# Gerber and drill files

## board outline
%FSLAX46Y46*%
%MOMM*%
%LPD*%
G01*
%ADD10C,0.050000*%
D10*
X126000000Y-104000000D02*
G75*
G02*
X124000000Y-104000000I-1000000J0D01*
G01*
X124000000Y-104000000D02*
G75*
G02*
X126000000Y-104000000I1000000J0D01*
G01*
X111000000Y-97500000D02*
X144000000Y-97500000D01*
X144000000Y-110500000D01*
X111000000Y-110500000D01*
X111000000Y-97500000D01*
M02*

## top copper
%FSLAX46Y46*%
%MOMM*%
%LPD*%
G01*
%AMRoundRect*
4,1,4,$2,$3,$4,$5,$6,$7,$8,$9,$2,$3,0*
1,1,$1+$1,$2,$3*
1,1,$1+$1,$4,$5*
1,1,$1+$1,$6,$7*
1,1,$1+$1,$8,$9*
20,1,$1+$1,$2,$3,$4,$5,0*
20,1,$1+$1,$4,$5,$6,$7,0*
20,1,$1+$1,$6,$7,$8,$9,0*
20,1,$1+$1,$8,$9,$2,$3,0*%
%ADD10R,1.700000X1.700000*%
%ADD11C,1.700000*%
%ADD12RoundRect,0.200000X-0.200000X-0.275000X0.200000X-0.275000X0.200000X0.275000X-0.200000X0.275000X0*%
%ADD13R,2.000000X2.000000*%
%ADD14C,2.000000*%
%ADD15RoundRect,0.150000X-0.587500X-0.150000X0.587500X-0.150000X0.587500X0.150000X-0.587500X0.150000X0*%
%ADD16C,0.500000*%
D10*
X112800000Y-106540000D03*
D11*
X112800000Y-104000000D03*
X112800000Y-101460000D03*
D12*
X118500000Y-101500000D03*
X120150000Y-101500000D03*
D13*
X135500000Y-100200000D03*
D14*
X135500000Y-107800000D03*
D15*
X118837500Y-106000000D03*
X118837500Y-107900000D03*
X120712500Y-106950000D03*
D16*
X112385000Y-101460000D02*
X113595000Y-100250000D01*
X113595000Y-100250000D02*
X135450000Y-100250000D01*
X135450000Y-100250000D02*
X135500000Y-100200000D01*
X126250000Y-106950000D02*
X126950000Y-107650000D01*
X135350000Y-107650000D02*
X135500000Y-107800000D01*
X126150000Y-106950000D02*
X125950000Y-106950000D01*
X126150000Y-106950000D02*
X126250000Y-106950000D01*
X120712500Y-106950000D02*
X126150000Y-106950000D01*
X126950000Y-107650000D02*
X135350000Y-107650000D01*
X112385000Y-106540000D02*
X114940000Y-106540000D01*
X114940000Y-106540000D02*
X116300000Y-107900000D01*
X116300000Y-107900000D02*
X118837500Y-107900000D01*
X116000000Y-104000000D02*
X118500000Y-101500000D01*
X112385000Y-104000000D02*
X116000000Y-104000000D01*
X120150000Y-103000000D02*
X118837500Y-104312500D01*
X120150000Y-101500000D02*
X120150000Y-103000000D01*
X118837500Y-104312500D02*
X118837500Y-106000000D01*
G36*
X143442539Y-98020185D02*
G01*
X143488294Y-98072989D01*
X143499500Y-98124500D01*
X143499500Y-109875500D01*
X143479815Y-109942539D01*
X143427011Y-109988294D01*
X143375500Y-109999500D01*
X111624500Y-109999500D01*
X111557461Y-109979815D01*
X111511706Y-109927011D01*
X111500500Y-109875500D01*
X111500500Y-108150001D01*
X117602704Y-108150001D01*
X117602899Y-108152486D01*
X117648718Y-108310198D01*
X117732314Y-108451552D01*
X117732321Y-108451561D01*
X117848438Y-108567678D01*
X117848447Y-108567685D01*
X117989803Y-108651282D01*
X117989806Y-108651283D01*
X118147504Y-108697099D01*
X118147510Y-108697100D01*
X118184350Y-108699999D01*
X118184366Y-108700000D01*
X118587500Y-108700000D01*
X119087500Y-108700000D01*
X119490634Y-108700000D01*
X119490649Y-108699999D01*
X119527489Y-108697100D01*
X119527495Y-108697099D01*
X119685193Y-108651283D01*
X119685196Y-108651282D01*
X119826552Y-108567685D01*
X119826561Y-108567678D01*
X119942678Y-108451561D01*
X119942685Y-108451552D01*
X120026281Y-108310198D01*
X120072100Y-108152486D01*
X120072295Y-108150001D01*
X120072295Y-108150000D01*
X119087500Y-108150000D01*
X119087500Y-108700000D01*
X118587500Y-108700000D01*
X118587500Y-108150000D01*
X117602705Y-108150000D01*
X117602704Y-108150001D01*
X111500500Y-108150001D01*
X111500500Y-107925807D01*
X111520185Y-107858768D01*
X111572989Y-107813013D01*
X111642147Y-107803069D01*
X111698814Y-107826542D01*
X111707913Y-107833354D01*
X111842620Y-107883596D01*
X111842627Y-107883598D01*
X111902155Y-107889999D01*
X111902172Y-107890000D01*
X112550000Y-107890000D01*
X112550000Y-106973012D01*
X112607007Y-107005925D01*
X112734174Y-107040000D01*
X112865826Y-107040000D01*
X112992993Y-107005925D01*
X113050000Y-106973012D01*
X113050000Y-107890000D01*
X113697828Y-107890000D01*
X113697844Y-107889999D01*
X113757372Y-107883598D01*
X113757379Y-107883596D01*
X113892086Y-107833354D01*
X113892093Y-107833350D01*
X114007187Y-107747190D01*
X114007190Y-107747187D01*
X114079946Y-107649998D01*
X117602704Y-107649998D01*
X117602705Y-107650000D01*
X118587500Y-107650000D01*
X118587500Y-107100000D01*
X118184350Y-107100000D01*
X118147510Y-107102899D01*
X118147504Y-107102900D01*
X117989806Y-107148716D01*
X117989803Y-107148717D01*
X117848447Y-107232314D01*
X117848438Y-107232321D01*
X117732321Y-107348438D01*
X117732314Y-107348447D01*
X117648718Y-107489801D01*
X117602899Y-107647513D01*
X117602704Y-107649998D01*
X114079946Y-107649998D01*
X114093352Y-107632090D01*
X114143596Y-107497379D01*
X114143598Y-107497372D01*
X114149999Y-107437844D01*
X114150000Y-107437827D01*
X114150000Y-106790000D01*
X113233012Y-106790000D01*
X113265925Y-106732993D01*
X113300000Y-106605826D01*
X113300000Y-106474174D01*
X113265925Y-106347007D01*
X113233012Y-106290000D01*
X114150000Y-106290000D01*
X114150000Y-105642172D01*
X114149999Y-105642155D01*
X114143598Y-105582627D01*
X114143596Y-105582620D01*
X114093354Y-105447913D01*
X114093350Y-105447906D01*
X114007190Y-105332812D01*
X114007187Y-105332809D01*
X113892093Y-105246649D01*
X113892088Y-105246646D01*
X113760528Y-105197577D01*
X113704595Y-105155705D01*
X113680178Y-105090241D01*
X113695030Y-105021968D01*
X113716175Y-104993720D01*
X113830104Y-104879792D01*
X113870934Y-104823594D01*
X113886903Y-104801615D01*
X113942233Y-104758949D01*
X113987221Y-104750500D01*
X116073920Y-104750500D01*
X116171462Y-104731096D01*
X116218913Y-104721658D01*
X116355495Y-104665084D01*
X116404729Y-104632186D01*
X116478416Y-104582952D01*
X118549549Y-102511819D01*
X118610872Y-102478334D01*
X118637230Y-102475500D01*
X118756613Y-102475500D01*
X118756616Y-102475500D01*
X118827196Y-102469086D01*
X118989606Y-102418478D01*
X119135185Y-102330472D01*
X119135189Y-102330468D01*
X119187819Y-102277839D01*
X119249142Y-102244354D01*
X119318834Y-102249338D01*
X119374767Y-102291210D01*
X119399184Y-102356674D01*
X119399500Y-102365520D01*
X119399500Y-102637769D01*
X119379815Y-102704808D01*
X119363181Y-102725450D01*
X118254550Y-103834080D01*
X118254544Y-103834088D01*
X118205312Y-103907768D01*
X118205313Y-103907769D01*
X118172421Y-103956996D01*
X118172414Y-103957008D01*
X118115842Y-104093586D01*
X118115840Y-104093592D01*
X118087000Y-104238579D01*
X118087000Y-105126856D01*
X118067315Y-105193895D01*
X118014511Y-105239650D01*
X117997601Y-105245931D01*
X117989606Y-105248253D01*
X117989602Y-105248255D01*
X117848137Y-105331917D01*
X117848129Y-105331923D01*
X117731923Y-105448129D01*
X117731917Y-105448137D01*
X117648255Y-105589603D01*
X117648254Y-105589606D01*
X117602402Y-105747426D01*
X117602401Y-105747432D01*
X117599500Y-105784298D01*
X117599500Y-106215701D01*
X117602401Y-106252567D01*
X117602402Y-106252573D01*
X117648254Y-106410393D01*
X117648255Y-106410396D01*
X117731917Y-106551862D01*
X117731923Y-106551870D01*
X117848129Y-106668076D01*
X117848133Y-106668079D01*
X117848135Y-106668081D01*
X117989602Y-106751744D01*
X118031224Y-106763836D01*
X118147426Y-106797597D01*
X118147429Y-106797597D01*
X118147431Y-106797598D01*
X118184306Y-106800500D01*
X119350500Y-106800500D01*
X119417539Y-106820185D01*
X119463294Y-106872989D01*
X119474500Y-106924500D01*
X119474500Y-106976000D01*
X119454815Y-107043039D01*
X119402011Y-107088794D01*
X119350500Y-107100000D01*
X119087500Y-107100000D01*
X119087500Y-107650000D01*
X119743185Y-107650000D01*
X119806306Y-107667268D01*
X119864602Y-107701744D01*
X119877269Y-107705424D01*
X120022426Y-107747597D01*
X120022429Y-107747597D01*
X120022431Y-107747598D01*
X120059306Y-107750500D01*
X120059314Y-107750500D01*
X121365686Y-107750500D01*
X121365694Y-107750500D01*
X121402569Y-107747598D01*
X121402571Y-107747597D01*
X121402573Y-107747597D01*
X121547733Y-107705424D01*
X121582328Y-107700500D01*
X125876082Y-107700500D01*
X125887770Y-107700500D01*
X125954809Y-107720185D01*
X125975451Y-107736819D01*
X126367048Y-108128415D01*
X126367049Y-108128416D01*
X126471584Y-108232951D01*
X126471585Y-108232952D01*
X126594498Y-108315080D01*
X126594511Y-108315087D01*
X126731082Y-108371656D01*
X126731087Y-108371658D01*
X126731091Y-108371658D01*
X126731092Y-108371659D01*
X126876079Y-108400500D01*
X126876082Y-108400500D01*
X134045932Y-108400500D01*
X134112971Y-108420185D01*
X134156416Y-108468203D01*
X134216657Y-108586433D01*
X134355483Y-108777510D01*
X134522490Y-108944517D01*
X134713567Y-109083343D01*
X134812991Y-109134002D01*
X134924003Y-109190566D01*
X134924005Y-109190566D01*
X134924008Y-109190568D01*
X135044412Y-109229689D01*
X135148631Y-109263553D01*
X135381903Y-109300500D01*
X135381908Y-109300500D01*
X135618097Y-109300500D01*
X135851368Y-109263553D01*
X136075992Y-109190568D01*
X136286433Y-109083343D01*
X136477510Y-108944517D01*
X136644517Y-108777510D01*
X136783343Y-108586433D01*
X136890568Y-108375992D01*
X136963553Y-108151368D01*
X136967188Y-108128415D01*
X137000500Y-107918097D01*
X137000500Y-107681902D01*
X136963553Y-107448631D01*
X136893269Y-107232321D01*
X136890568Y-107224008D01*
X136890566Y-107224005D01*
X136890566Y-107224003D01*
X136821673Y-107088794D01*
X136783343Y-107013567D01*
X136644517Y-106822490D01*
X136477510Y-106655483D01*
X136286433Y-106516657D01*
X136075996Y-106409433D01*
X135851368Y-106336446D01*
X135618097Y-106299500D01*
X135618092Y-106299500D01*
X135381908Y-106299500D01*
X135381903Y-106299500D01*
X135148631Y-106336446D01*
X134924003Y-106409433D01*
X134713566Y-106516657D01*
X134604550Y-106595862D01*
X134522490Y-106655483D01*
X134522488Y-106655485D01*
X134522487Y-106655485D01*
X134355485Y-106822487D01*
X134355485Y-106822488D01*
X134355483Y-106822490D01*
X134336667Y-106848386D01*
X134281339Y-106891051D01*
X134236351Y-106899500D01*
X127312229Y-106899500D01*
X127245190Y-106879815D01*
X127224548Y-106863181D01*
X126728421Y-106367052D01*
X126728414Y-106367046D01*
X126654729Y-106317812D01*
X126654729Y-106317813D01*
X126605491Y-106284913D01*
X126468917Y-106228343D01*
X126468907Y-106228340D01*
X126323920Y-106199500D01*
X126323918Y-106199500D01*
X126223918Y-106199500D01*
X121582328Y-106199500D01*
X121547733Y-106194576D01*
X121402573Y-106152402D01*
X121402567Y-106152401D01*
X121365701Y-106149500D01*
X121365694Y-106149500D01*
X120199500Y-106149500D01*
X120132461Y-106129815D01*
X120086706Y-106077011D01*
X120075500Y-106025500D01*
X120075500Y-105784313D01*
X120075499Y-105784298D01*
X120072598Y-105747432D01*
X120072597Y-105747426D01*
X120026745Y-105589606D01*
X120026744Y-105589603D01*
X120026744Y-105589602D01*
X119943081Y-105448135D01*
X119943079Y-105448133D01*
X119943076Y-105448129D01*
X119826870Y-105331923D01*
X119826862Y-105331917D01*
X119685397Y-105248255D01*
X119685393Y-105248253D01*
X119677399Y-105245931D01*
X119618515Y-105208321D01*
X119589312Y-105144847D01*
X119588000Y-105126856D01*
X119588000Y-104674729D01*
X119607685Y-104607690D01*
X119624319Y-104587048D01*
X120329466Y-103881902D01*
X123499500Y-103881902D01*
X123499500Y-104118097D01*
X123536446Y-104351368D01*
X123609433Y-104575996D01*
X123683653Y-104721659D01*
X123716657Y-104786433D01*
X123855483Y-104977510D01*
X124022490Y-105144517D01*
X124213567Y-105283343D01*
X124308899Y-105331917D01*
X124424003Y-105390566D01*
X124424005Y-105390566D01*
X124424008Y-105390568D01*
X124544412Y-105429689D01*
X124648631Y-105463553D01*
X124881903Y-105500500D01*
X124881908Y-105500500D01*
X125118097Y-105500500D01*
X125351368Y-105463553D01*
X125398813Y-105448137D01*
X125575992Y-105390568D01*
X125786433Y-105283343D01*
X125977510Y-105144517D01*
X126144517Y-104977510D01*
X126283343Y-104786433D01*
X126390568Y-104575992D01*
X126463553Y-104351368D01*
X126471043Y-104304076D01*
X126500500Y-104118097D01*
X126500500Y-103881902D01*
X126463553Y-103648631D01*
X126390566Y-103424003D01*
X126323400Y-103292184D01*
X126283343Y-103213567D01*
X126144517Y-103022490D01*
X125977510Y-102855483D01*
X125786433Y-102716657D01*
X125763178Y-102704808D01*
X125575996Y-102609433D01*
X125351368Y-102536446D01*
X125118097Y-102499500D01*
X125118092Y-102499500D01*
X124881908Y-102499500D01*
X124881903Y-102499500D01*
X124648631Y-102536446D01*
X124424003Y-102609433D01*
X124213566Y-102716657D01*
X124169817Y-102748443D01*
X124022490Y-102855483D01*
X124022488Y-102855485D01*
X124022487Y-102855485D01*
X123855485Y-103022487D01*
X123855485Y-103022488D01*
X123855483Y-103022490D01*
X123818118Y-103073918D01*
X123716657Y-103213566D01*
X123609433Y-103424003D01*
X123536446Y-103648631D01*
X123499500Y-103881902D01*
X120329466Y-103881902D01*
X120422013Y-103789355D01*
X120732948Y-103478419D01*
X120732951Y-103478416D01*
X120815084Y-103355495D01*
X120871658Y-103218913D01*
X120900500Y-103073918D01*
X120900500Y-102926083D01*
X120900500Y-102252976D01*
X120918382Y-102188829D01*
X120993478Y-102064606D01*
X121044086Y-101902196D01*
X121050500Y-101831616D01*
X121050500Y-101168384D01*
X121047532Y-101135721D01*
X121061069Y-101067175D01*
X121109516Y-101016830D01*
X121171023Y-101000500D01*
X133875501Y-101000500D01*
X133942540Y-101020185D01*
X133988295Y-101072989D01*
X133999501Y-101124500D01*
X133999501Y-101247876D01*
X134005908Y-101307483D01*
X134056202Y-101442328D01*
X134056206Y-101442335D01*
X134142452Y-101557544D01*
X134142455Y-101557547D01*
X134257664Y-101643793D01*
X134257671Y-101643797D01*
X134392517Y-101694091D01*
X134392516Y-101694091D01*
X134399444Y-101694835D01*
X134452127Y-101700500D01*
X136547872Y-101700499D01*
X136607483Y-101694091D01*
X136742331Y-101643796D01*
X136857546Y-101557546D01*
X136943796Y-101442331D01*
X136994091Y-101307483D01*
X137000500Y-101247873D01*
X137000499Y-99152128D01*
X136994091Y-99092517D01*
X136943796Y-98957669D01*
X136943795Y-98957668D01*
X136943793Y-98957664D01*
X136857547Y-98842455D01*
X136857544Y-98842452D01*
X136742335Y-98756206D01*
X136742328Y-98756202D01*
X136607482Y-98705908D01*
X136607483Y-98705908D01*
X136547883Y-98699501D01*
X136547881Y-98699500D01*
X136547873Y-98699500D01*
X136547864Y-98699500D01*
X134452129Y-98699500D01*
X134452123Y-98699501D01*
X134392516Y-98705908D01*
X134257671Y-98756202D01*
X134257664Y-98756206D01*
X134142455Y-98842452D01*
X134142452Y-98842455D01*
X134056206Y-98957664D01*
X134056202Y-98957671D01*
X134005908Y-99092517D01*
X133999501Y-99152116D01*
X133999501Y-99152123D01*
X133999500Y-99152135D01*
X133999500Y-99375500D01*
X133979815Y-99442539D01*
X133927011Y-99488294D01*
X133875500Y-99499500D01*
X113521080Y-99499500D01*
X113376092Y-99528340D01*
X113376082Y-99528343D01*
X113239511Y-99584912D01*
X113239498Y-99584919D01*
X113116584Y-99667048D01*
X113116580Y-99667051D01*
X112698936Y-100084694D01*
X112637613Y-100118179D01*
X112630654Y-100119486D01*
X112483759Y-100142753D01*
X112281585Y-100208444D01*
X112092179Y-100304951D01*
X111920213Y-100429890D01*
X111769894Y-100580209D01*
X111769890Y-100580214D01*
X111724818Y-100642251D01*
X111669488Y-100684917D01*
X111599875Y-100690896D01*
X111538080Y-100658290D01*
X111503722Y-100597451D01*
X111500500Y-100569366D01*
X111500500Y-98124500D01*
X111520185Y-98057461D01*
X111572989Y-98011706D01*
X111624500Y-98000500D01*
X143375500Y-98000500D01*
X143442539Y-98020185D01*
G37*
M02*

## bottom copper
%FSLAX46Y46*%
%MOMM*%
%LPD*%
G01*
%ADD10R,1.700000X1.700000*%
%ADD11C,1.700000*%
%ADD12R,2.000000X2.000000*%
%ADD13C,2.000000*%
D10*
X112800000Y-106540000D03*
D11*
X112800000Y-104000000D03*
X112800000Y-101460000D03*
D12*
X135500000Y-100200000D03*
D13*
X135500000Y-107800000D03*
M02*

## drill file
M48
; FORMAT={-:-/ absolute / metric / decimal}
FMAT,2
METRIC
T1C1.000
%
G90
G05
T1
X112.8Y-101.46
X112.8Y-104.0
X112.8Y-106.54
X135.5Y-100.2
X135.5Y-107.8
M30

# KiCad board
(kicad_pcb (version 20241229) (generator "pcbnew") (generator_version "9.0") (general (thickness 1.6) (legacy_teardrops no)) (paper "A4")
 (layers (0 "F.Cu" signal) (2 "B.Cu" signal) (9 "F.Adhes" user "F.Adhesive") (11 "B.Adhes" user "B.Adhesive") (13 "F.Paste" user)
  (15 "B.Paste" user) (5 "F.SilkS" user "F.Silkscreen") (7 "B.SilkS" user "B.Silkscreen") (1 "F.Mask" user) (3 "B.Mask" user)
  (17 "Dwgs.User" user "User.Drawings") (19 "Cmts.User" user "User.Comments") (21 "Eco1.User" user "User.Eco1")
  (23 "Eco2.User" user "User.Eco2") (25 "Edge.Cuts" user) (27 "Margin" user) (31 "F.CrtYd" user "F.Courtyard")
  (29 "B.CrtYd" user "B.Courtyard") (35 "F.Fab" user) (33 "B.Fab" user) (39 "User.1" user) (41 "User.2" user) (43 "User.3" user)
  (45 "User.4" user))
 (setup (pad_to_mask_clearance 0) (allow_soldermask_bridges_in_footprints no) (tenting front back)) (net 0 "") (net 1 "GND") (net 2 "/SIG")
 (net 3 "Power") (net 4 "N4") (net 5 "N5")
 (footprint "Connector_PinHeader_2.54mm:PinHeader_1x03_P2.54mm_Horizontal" (layer "F.Cu") (at 112.8 106.54 180)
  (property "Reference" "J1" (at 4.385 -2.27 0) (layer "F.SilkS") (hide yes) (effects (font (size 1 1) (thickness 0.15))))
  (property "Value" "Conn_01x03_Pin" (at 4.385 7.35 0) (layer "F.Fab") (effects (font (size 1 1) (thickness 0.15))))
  (pad "1" thru_hole rect (at 0 0 180) (size 1.7 1.7) (drill 1) (layers "*.Cu" "*.Mask") (remove_unused_layers no) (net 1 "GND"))
  (pad "2" thru_hole circle (at 0 2.54 180) (size 1.7 1.7) (drill 1) (layers "*.Cu" "*.Mask") (remove_unused_layers no) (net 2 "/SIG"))
  (pad "3" thru_hole circle (at 0 5.08 180) (size 1.7 1.7) (drill 1) (layers "*.Cu" "*.Mask") (remove_unused_layers no) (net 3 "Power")))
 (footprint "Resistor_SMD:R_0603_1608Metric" (layer "F.Cu") (at 119.325 101.5)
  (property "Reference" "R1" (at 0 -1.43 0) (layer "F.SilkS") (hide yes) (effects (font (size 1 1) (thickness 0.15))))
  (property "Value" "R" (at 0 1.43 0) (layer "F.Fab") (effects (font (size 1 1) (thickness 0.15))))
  (pad "1" smd roundrect (at -0.825 0) (size 0.8 0.95) (layers "F.Cu" "F.Mask" "F.Paste") (roundrect_rratio 0.25) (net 2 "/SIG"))
  (pad "2" smd roundrect (at 0.825 0) (size 0.8 0.95) (layers "F.Cu" "F.Mask" "F.Paste") (roundrect_rratio 0.25) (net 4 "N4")))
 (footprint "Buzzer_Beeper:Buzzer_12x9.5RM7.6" (layer "F.Cu") (at 135.5 100.2 -90)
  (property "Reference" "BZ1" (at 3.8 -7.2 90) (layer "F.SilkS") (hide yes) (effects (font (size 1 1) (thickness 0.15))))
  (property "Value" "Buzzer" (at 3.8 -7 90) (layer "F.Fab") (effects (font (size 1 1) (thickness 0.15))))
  (pad "1" thru_hole rect (at 0 0 270) (size 2 2) (drill 1) (layers "*.Cu" "*.Mask") (remove_unused_layers no) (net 3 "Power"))
  (pad "2" thru_hole circle (at 7.6 0 270) (size 2 2) (drill 1) (layers "*.Cu" "*.Mask") (remove_unused_layers no) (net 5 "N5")))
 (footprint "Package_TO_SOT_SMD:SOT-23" (layer "F.Cu") (at 119.775 106.95)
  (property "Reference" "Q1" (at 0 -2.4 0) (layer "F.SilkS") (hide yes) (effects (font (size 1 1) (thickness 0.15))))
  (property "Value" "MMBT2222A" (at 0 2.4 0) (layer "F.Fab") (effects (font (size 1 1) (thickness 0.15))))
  (pad "1" smd roundrect (at -0.9375 -0.95) (size 1.475 0.6) (layers "F.Cu" "F.Mask" "F.Paste") (roundrect_rratio 0.25) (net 4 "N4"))
  (pad "2" smd roundrect (at -0.9375 0.95) (size 1.475 0.6) (layers "F.Cu" "F.Mask" "F.Paste") (roundrect_rratio 0.25) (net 1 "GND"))
  (pad "3" smd roundrect (at 0.9375 0) (size 1.475 0.6) (layers "F.Cu" "F.Mask" "F.Paste") (roundrect_rratio 0.25) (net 5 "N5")))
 (gr_circle (center 125 104) (end 126 104) (stroke (width 0.05) (type default)) (fill no) (layer "Edge.Cuts"))
 (gr_rect (start 111 97.5) (end 144 110.5) (stroke (width 0.05) (type default)) (fill no) (layer "Edge.Cuts"))
 (segment (start 112.385 101.46) (end 113.595 100.25) (width 0.5) (layer "F.Cu") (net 3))
 (segment (start 113.595 100.25) (end 135.45 100.25) (width 0.5) (layer "F.Cu") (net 3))
 (segment (start 135.45 100.25) (end 135.5 100.2) (width 0.5) (layer "F.Cu") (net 3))
 (segment (start 126.25 106.95) (end 126.95 107.65) (width 0.5) (layer "F.Cu") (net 5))
 (segment (start 135.35 107.65) (end 135.5 107.8) (width 0.5) (layer "F.Cu") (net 5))
 (segment (start 126.15 106.95) (end 125.95 106.95) (width 0.5) (layer "F.Cu") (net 5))
 (segment (start 126.15 106.95) (end 126.25 106.95) (width 0.5) (layer "F.Cu") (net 5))
 (segment (start 120.7125 106.95) (end 126.15 106.95) (width 0.5) (layer "F.Cu") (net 5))
 (segment (start 126.95 107.65) (end 135.35 107.65) (width 0.5) (layer "F.Cu") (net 5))
 (segment (start 112.385 106.54) (end 114.94 106.54) (width 0.5) (layer "F.Cu") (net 1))
 (segment (start 114.94 106.54) (end 116.3 107.9) (width 0.5) (layer "F.Cu") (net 1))
 (segment (start 116.3 107.9) (end 118.8375 107.9) (width 0.5) (layer "F.Cu") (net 1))
 (segment (start 116 104) (end 118.5 101.5) (width 0.5) (layer "F.Cu") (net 2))
 (segment (start 112.385 104) (end 116 104) (width 0.5) (layer "F.Cu") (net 2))
 (segment (start 120.15 103) (end 118.8375 104.3125) (width 0.5) (layer "F.Cu") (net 4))
 (segment (start 120.15 101.5) (end 120.15 103) (width 0.5) (layer "F.Cu") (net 4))
 (segment (start 118.8375 104.3125) (end 118.8375 106) (width 0.5) (layer "F.Cu") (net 4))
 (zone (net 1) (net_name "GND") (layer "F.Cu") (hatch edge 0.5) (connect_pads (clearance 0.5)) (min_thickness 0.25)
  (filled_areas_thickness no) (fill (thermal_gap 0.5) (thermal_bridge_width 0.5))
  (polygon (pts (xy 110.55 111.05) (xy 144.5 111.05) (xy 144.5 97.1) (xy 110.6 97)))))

